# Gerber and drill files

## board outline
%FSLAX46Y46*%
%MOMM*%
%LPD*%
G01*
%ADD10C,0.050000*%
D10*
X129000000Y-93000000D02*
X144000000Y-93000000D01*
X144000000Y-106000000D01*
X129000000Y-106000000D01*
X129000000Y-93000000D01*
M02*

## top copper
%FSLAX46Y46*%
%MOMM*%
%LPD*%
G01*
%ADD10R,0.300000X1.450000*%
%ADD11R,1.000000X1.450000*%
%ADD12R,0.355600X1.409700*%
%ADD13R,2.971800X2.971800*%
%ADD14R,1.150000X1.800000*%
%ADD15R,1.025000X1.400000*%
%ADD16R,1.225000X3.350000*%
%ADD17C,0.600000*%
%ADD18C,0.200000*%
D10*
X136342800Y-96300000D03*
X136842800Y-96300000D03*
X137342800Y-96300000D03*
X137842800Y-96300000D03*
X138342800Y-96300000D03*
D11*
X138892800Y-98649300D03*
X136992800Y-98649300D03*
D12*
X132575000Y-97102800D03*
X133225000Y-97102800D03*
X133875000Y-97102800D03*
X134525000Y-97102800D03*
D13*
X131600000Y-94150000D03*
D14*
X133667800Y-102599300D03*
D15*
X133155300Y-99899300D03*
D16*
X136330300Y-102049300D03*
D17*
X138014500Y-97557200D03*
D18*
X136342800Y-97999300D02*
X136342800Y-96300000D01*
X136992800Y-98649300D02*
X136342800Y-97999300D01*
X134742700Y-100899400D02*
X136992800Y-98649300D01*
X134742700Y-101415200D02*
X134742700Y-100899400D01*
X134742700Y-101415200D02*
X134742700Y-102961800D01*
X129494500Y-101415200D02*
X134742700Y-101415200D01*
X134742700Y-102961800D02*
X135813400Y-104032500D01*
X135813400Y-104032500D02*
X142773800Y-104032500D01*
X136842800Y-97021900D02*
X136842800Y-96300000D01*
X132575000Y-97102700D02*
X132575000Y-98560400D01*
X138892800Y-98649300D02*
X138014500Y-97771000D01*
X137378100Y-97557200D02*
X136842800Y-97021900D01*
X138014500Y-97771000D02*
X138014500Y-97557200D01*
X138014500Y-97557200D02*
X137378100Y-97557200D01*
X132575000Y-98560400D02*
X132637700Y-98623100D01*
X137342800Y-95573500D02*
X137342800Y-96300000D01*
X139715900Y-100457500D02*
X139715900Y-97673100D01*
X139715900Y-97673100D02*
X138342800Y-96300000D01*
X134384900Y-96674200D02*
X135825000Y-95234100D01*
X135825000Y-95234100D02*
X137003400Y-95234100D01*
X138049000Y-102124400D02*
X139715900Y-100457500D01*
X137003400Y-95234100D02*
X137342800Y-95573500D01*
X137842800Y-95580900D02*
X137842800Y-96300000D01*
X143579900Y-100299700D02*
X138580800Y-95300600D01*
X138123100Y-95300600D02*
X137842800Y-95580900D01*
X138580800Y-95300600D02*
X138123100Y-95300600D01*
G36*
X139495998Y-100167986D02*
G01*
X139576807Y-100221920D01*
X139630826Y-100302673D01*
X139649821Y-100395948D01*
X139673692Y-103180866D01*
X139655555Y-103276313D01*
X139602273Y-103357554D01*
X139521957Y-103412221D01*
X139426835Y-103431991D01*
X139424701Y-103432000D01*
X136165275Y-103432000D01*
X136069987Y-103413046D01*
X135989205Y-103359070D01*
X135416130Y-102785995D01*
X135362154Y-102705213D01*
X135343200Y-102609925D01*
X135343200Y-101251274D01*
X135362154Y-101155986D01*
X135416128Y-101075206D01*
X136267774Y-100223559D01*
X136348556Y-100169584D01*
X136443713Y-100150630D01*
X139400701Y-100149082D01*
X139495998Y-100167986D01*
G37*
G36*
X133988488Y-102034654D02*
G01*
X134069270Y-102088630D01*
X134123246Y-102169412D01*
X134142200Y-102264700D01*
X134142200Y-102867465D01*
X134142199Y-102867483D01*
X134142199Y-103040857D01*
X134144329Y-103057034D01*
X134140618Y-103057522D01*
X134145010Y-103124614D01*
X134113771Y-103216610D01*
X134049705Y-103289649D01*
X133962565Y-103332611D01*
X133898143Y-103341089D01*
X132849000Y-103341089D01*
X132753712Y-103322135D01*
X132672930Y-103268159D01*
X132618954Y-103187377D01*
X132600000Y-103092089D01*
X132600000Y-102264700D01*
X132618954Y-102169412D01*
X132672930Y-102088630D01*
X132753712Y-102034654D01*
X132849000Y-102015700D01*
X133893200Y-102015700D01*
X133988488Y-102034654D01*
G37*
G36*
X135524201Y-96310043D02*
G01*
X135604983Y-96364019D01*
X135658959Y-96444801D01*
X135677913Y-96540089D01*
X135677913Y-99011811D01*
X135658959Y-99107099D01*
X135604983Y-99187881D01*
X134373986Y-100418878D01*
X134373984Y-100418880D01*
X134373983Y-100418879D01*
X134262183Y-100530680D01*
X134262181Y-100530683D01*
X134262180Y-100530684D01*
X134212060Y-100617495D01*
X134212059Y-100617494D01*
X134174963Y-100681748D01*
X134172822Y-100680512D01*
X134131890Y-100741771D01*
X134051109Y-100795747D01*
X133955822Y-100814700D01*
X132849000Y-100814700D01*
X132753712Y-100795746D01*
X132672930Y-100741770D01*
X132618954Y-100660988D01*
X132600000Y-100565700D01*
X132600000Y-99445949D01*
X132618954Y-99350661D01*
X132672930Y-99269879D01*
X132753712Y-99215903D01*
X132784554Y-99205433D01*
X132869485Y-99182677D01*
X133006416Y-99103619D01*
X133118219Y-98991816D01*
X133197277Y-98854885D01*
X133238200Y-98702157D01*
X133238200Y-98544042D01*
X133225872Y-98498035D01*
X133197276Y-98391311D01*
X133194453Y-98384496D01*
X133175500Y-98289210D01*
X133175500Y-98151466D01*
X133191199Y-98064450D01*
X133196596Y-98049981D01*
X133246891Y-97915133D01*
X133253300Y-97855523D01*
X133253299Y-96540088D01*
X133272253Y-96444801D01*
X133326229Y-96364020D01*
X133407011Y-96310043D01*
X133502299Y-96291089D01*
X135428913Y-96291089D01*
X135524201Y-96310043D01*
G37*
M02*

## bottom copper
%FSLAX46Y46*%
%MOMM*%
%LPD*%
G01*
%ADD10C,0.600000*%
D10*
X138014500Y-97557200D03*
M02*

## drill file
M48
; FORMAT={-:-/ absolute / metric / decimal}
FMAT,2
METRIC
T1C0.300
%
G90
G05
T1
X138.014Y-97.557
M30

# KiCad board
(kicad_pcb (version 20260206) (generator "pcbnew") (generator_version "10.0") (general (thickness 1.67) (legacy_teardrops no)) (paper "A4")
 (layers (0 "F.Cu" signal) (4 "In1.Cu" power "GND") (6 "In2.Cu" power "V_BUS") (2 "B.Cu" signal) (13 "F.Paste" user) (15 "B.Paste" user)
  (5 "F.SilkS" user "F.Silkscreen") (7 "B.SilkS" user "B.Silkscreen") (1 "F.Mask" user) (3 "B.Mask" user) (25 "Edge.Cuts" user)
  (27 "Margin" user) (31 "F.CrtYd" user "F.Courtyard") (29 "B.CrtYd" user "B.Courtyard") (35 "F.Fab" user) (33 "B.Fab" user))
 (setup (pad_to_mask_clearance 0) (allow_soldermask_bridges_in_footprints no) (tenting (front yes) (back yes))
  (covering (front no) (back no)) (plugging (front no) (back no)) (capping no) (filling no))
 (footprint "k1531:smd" (layer "F.Cu") (at 136.3428 96.3)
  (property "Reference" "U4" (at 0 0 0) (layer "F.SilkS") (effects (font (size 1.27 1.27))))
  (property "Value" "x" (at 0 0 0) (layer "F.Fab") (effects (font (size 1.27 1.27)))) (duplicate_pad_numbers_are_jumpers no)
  (pad "1" smd rect (at 0 0) (size 0.3 1.45) (layers "F.Cu" "F.Mask") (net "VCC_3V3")))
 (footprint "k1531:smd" (layer "F.Cu") (at 136.8428 96.3)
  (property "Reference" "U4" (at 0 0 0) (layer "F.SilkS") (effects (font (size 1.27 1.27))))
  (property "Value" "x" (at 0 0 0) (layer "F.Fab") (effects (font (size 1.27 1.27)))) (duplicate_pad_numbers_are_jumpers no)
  (pad "1" smd rect (at 0 0) (size 0.3 1.45) (layers "F.Cu" "F.Mask") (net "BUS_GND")))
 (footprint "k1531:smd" (layer "F.Cu") (at 137.3428 96.3)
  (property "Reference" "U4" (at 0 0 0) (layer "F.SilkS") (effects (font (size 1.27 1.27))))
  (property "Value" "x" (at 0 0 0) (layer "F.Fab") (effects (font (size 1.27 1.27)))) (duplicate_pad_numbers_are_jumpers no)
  (pad "1" smd rect (at 0 0) (size 0.3 1.45) (layers "F.Cu" "F.Mask") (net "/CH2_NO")))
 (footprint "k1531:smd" (layer "F.Cu") (at 137.8428 96.3)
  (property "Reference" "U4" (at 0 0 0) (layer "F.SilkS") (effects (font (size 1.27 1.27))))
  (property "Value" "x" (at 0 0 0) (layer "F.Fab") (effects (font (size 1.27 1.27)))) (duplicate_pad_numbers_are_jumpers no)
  (pad "1" smd rect (at 0 0) (size 0.3 1.45) (layers "F.Cu" "F.Mask") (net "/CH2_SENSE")))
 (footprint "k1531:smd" (layer "F.Cu") (at 138.3428 96.3)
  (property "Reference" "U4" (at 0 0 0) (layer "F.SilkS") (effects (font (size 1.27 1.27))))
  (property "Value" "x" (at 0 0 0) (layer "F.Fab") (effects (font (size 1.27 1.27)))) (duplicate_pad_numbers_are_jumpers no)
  (pad "1" smd rect (at 0 0) (size 0.3 1.45) (layers "F.Cu" "F.Mask") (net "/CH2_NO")))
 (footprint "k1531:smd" (layer "F.Cu") (at 138.8928 98.6493)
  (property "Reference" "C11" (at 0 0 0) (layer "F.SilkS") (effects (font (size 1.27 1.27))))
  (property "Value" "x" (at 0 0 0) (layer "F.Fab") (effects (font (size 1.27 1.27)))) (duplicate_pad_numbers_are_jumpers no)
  (pad "1" smd rect (at 0 0) (size 1 1.45) (layers "F.Cu" "F.Mask") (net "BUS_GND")))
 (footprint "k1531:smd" (layer "F.Cu") (at 136.9928 98.6493)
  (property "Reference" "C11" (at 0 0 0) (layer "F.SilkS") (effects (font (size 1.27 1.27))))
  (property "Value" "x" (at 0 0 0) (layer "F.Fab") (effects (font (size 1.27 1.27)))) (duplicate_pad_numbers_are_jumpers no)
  (pad "1" smd rect (at 0 0) (size 1 1.45) (layers "F.Cu" "F.Mask") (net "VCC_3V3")))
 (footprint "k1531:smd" (layer "F.Cu") (at 132.575 97.1028)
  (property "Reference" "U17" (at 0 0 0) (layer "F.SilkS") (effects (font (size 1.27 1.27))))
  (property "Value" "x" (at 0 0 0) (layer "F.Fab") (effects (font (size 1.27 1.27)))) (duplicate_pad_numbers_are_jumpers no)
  (pad "1" smd rect (at 0 0) (size 0.3556 1.4097) (layers "F.Cu" "F.Mask") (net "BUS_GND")))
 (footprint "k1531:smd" (layer "F.Cu") (at 133.225 97.1028)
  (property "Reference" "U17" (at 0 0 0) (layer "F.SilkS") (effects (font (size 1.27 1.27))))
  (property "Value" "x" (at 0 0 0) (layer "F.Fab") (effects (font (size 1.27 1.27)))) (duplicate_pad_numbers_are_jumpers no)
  (pad "1" smd rect (at 0 0) (size 0.3556 1.4097) (layers "F.Cu" "F.Mask") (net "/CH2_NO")))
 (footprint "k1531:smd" (layer "F.Cu") (at 133.875 97.1028)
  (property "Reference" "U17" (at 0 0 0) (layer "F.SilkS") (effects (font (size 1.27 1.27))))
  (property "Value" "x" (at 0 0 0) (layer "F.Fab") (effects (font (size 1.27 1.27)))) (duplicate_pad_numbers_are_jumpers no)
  (pad "1" smd rect (at 0 0) (size 0.3556 1.4097) (layers "F.Cu" "F.Mask") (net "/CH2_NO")))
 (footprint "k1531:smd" (layer "F.Cu") (at 134.525 97.1028)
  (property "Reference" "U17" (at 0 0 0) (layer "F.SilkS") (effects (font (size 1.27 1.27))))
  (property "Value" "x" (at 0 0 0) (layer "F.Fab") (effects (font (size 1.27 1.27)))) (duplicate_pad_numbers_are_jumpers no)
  (pad "1" smd rect (at 0 0) (size 0.3556 1.4097) (layers "F.Cu" "F.Mask") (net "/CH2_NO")))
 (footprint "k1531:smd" (layer "F.Cu") (at 131.6 94.15)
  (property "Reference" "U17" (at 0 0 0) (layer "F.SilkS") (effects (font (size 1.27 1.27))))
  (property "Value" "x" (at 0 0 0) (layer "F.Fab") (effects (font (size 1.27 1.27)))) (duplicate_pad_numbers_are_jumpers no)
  (pad "1" smd rect (at 0 0) (size 2.9718 2.9718) (layers "F.Cu" "F.Mask") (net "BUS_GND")))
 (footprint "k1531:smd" (layer "F.Cu") (at 133.6678 102.5993)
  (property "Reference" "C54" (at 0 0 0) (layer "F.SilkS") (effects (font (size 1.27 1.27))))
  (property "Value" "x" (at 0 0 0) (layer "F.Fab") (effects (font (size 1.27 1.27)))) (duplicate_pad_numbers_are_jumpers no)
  (pad "1" smd rect (at 0 0) (size 1.15 1.8) (layers "F.Cu" "F.Mask") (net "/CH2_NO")))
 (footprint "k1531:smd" (layer "F.Cu") (at 133.1553 99.8993)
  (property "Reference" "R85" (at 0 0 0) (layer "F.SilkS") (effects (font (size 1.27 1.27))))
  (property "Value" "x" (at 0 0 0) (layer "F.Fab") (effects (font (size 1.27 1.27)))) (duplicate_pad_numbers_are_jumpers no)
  (pad "1" smd rect (at 0 0) (size 1.025 1.4) (layers "F.Cu" "F.Mask") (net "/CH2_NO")))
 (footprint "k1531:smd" (layer "F.Cu") (at 136.3303 102.0493)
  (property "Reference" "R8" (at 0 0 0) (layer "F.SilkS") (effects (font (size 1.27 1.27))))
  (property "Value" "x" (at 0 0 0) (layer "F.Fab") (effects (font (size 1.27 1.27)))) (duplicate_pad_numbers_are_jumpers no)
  (pad "1" smd rect (at 0 0) (size 1.225 3.35) (layers "F.Cu" "F.Mask") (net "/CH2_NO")))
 (gr_rect (start 129 93) (end 144 106) (stroke (width 0.05) (type default)) (fill no) (layer "Edge.Cuts"))
 (segment (start 136.3428 97.9993) (end 136.3428 96.3) (width 0.2) (layer "F.Cu") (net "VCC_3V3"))
 (segment (start 136.9928 98.6493) (end 136.3428 97.9993) (width 0.2) (layer "F.Cu") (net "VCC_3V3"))
 (segment (start 134.7427 100.8994) (end 136.9928 98.6493) (width 0.2) (layer "F.Cu") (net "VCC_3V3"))
 (segment (start 134.7427 101.4152) (end 134.7427 100.8994) (width 0.2) (layer "F.Cu") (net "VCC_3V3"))
 (segment (start 134.7427 101.4152) (end 134.7427 102.9618) (width 0.2) (layer "F.Cu") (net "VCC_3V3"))
 (segment (start 129.4945 101.4152) (end 134.7427 101.4152) (width 0.2) (layer "F.Cu") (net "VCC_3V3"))
 (segment (start 134.7427 102.9618) (end 135.8134 104.0325) (width 0.2) (layer "F.Cu") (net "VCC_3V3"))
 (segment (start 135.8134 104.0325) (end 142.7738 104.0325) (width 0.2) (layer "F.Cu") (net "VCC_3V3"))
 (segment (start 136.8428 97.0219) (end 136.8428 96.3) (width 0.2) (layer "F.Cu") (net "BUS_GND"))
 (segment (start 132.575 97.1027) (end 132.575 98.5604) (width 0.2) (layer "F.Cu") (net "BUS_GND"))
 (segment (start 138.8928 98.6493) (end 138.0145 97.771) (width 0.2) (layer "F.Cu") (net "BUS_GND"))
 (segment (start 137.3781 97.5572) (end 136.8428 97.0219) (width 0.2) (layer "F.Cu") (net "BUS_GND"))
 (segment (start 138.0145 97.771) (end 138.0145 97.5572) (width 0.2) (layer "F.Cu") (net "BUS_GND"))
 (segment (start 138.0145 97.5572) (end 137.3781 97.5572) (width 0.2) (layer "F.Cu") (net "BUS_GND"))
 (segment (start 132.575 98.5604) (end 132.6377 98.6231) (width 0.2) (layer "F.Cu") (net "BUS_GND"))
 (via (at 138.0145 97.5572) (size 0.6) (drill 0.3) (layers "F.Cu" "B.Cu") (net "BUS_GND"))
 (segment (start 137.3428 95.5735) (end 137.3428 96.3) (width 0.2) (layer "F.Cu") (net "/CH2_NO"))
 (segment (start 139.7159 100.4575) (end 139.7159 97.6731) (width 0.2) (layer "F.Cu") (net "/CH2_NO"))
 (segment (start 139.7159 97.6731) (end 138.3428 96.3) (width 0.2) (layer "F.Cu") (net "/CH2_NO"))
 (segment (start 134.3849 96.6742) (end 135.825 95.2341) (width 0.2) (layer "F.Cu") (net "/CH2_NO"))
 (segment (start 135.825 95.2341) (end 137.0034 95.2341) (width 0.2) (layer "F.Cu") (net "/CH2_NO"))
 (segment (start 138.049 102.1244) (end 139.7159 100.4575) (width 0.2) (layer "F.Cu") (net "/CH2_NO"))
 (segment (start 137.0034 95.2341) (end 137.3428 95.5735) (width 0.2) (layer "F.Cu") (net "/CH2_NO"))
 (segment (start 137.8428 95.5809) (end 137.8428 96.3) (width 0.2) (layer "F.Cu") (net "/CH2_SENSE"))
 (segment (start 143.5799 100.2997) (end 138.5808 95.3006) (width 0.2) (layer "F.Cu") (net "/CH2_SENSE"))
 (segment (start 138.1231 95.3006) (end 137.8428 95.5809) (width 0.2) (layer "F.Cu") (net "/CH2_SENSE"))
 (segment (start 138.5808 95.3006) (end 138.1231 95.3006) (width 0.2) (layer "F.Cu") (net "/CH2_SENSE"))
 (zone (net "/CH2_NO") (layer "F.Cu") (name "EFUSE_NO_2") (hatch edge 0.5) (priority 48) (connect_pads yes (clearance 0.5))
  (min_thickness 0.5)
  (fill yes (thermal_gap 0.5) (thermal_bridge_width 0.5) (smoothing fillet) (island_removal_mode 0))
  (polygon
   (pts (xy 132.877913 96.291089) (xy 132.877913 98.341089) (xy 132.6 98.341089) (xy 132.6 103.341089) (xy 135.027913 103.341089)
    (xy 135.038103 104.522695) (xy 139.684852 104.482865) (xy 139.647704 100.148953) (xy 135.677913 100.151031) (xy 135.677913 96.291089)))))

